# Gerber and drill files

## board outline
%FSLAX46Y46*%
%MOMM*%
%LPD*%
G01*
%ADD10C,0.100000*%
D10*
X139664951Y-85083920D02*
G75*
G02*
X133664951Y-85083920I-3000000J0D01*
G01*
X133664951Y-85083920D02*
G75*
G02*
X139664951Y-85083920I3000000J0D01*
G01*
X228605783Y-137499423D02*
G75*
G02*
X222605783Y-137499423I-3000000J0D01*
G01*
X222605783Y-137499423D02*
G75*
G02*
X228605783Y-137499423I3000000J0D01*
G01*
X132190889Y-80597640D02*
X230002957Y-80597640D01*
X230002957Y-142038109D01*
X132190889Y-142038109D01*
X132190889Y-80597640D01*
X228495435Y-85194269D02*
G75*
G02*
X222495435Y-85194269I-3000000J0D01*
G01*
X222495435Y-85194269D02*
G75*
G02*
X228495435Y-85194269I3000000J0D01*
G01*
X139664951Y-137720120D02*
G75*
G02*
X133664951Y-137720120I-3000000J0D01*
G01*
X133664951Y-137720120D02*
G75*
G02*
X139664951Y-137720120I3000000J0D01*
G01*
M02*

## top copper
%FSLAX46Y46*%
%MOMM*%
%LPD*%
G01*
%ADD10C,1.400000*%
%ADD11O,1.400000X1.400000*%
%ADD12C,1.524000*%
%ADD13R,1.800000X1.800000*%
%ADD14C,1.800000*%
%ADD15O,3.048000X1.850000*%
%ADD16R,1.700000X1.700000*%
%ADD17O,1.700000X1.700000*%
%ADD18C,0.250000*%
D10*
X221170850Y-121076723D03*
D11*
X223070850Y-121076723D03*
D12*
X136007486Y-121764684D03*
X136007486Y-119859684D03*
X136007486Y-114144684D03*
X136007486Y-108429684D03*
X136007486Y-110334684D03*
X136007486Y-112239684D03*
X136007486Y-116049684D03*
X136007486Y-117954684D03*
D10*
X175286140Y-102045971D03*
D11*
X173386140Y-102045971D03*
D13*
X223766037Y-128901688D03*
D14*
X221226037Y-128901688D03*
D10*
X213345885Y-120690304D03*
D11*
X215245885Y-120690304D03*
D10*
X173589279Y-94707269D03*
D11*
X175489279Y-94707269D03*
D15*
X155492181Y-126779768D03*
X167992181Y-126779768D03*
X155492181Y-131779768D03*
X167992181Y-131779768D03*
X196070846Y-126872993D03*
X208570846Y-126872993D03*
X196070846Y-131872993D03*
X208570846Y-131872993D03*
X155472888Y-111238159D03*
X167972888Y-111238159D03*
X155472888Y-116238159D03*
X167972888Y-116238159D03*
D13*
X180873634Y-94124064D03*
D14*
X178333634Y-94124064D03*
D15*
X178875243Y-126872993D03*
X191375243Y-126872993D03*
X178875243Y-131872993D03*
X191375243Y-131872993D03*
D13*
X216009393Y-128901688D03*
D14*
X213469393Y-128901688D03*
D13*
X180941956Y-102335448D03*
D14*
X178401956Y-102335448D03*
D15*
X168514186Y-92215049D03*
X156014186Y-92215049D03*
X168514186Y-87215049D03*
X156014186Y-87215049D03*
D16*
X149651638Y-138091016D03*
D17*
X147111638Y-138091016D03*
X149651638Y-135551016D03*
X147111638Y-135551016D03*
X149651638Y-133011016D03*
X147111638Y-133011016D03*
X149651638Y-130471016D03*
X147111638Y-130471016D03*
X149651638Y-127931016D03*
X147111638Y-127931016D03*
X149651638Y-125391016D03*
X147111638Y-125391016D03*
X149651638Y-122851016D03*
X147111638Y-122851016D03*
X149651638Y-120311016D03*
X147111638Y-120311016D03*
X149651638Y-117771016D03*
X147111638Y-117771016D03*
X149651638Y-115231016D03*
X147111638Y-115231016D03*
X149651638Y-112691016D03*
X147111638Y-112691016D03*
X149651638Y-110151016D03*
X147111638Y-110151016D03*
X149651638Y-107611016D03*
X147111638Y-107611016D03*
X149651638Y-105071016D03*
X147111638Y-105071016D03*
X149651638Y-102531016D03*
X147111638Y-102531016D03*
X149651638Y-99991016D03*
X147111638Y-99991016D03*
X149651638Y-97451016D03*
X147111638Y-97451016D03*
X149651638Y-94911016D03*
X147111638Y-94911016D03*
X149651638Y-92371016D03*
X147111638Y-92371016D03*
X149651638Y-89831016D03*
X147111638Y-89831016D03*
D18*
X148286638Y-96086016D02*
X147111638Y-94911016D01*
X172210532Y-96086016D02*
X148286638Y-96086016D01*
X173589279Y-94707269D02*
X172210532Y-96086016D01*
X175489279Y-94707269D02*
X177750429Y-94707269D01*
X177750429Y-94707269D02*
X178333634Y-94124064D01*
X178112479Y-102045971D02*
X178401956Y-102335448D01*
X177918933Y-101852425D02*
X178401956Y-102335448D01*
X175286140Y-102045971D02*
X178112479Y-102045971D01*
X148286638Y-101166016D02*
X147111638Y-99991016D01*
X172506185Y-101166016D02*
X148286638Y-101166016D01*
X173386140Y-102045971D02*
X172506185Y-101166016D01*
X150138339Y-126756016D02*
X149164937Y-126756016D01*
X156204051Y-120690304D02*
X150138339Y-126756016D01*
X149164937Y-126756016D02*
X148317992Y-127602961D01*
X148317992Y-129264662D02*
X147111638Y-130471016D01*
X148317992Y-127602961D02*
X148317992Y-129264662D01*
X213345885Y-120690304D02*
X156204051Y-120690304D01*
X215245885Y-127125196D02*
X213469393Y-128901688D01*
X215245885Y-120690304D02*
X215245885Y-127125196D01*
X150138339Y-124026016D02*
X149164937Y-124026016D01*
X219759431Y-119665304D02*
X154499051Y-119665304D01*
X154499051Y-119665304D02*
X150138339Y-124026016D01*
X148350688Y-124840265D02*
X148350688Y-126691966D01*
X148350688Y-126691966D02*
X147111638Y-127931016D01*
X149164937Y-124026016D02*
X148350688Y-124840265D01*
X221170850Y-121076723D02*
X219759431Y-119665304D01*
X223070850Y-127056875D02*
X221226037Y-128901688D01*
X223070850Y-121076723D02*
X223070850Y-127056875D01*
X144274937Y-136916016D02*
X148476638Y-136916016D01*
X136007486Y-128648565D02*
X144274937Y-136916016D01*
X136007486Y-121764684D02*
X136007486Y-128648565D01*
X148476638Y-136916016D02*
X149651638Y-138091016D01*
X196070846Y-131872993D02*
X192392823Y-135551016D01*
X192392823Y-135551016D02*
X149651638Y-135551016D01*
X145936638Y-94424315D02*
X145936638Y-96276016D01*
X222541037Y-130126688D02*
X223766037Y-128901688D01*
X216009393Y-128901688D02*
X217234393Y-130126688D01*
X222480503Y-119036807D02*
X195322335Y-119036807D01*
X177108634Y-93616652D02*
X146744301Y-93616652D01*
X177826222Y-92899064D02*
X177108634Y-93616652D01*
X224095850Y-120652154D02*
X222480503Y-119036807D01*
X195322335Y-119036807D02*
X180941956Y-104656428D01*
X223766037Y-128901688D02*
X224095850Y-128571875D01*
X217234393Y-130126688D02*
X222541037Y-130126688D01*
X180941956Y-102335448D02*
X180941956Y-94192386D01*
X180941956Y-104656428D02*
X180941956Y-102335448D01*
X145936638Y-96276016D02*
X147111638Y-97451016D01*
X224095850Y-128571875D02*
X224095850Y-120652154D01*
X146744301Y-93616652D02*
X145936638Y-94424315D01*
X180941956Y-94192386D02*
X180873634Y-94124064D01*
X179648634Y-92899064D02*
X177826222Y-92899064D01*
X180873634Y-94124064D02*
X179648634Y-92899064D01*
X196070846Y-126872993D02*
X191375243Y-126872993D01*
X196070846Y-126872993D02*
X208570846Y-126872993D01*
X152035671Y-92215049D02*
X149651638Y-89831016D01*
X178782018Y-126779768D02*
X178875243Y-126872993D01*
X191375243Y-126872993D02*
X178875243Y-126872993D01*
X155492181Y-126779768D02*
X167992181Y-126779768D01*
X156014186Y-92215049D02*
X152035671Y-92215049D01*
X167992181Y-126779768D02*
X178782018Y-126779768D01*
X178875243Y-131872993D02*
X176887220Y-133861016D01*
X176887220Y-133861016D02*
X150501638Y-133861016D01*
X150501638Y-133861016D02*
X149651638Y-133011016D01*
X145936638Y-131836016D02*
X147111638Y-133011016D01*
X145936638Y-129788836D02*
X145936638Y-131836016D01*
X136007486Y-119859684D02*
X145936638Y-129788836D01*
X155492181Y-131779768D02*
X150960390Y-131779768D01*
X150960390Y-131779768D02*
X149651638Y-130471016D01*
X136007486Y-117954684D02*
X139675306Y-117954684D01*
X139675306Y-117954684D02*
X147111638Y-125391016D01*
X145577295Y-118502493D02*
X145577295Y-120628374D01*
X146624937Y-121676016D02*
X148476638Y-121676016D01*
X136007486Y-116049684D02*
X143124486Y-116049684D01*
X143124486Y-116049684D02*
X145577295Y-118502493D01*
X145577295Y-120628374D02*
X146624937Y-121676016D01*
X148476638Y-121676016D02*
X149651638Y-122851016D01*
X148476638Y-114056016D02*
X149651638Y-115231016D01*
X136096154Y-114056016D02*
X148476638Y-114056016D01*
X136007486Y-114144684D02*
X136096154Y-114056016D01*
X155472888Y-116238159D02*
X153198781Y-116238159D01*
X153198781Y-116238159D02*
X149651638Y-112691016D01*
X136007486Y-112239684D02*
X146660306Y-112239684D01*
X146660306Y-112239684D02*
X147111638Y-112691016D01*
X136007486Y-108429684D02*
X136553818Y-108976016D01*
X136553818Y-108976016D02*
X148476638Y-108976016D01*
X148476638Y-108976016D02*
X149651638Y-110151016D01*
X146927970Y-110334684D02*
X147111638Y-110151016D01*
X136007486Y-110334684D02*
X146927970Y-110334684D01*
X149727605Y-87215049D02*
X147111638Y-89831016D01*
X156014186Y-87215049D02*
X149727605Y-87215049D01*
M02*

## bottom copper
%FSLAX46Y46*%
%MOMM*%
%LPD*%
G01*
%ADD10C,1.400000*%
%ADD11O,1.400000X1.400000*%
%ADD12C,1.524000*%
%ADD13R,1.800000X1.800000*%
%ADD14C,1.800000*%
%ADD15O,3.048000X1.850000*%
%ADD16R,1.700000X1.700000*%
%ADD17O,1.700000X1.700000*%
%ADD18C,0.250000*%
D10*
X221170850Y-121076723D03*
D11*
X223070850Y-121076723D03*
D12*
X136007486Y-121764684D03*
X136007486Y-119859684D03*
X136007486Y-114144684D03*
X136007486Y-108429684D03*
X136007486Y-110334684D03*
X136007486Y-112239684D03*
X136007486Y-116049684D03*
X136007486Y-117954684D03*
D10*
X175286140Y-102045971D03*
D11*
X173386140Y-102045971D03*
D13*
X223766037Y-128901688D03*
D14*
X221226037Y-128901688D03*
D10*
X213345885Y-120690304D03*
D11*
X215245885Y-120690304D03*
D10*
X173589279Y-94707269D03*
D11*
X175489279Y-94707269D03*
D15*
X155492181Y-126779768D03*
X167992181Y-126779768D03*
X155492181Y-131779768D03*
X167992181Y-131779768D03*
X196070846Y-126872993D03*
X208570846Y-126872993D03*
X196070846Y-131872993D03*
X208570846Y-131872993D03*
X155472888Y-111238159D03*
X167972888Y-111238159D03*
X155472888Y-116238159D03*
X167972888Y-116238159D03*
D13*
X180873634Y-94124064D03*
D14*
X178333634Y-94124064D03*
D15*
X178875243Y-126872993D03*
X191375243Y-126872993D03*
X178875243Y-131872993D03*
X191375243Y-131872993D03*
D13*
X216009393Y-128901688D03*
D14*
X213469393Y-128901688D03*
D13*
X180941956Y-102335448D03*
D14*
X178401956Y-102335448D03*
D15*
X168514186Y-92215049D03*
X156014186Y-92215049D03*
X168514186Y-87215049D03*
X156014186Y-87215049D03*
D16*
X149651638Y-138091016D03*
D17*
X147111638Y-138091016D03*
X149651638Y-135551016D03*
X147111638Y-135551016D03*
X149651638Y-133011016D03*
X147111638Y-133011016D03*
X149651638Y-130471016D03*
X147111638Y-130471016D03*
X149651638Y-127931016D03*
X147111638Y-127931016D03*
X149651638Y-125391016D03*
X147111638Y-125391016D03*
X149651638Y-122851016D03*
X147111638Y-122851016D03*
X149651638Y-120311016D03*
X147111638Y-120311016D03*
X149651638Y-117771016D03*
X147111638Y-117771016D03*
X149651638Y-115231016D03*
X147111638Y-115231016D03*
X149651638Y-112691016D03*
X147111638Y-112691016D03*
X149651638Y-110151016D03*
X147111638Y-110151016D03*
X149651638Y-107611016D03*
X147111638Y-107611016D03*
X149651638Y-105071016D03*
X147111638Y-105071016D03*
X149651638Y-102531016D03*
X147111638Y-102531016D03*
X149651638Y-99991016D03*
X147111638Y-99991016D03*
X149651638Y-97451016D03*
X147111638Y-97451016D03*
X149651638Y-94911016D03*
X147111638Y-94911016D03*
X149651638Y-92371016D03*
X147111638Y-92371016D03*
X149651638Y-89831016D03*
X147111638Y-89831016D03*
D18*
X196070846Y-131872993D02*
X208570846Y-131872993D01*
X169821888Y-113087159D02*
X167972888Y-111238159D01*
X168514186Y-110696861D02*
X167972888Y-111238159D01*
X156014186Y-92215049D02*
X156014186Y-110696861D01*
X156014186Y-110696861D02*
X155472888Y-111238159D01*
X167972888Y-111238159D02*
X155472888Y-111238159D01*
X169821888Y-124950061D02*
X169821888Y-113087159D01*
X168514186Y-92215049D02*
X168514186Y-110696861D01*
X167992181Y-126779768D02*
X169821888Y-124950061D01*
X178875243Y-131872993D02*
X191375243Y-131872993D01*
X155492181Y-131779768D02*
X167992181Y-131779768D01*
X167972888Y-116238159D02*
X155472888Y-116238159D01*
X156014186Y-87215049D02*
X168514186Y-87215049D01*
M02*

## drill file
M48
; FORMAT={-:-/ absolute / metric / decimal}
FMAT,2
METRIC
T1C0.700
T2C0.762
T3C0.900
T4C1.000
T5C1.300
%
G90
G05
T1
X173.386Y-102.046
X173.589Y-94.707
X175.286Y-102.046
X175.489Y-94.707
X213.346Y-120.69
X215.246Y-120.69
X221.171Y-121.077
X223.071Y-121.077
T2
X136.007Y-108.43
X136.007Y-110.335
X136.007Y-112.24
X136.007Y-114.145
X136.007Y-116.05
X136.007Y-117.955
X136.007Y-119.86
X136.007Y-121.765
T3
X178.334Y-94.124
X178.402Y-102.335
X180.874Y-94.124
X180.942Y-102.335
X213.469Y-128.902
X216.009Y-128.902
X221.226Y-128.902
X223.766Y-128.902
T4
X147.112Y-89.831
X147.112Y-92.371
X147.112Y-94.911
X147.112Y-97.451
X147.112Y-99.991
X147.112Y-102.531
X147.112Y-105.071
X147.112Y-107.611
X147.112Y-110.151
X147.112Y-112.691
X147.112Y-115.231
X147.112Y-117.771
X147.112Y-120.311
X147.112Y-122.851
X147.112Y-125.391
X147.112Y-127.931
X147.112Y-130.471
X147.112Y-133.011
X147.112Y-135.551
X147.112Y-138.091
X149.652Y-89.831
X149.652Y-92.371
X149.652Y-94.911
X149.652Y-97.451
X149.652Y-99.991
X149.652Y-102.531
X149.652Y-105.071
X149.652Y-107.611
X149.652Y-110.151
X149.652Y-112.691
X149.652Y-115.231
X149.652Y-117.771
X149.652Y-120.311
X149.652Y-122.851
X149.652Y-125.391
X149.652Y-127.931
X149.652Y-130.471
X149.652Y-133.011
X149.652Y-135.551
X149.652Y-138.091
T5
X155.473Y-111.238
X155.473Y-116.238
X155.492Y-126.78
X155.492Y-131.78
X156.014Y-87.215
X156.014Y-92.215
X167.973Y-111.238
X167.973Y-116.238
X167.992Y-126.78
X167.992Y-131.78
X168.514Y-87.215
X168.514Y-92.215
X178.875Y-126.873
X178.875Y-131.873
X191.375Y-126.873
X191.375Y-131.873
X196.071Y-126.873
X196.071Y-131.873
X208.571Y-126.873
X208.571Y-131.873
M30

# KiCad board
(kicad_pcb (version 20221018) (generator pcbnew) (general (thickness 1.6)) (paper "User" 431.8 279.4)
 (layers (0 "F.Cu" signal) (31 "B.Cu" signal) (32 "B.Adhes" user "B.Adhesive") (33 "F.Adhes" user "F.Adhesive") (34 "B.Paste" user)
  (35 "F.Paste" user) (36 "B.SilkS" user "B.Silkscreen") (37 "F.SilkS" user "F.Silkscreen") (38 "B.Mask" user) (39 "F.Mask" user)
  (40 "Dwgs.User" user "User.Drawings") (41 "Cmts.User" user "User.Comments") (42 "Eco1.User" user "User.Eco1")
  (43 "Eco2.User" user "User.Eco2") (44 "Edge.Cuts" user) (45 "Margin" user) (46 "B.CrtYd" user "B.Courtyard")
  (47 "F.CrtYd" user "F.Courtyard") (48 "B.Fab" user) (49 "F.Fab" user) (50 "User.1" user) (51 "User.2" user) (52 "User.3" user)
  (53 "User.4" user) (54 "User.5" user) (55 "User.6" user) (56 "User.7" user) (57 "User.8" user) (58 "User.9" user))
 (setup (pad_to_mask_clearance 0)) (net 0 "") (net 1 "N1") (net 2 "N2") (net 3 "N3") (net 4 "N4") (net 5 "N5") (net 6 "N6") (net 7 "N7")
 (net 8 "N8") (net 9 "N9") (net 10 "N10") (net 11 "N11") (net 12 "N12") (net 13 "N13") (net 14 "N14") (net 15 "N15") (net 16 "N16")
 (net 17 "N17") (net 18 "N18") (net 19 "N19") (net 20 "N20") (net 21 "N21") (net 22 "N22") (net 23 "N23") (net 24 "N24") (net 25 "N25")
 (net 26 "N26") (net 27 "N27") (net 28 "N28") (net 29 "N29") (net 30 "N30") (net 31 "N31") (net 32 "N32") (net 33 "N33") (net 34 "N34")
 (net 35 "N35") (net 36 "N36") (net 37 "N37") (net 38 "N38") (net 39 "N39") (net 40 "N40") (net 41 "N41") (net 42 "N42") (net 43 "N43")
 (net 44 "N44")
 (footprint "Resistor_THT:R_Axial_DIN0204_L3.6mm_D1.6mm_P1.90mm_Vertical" (layer "F.Cu") (at 221.17085 121.076723)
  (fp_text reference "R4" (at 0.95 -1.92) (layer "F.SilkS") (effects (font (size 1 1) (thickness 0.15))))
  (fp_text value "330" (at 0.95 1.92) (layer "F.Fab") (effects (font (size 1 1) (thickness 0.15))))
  (pad "1" thru_hole circle (at 0 0) (size 1.4 1.4) (drill 0.7) (layers "*.Cu" "*.Mask") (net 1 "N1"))
  (pad "2" thru_hole oval (at 1.9 0) (size 1.4 1.4) (drill 0.7) (layers "*.Cu" "*.Mask") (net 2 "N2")))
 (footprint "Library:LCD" (layer "F.Cu") (at 136.007486 117.319684)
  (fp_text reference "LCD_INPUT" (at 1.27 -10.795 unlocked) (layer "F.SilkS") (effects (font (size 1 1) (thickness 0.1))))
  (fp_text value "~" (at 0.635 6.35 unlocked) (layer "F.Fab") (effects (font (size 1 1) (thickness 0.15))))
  (pad "1" thru_hole circle (at 0 4.445) (size 1.524 1.524) (drill 0.762) (layers "*.Cu" "*.Mask") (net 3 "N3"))
  (pad "2" thru_hole circle (at 0 2.54) (size 1.524 1.524) (drill 0.762) (layers "*.Cu" "*.Mask") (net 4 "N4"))
  (pad "3" thru_hole circle (at 0 -3.175) (size 1.524 1.524) (drill 0.762) (layers "*.Cu" "*.Mask") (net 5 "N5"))
  (pad "4" thru_hole circle (at 0 -8.89) (size 1.524 1.524) (drill 0.762) (layers "*.Cu" "*.Mask") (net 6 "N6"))
  (pad "5" thru_hole circle (at 0 -6.985) (size 1.524 1.524) (drill 0.762) (layers "*.Cu" "*.Mask") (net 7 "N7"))
  (pad "6" thru_hole circle (at 0 -5.08) (size 1.524 1.524) (drill 0.762) (layers "*.Cu" "*.Mask") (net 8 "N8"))
  (pad "7" thru_hole circle (at 0 -1.27) (size 1.524 1.524) (drill 0.762) (layers "*.Cu" "*.Mask") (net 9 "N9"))
  (pad "8" thru_hole circle (at 0 0.635) (size 1.524 1.524) (drill 0.762) (layers "*.Cu" "*.Mask") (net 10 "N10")))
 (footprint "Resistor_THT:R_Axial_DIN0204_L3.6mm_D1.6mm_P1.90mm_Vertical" (layer "F.Cu") (at 175.28614 102.045971 180)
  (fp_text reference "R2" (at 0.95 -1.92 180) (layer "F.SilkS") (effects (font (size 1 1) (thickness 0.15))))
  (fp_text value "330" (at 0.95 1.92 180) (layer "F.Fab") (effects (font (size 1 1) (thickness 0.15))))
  (pad "1" thru_hole circle (at 0 0 180) (size 1.4 1.4) (drill 0.7) (layers "*.Cu" "*.Mask") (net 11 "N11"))
  (pad "2" thru_hole oval (at 1.9 0 180) (size 1.4 1.4) (drill 0.7) (layers "*.Cu" "*.Mask") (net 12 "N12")))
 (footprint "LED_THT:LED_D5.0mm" (layer "F.Cu") (at 223.766037 128.901688 180)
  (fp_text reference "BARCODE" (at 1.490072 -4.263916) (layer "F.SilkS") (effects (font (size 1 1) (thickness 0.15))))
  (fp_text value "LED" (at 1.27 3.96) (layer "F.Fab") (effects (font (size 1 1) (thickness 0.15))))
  (pad "1" thru_hole rect (at 0 0 180) (size 1.8 1.8) (drill 0.9) (layers "*.Cu" "*.Mask") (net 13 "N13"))
  (pad "2" thru_hole circle (at 2.54 0 180) (size 1.8 1.8) (drill 0.9) (layers "*.Cu" "*.Mask") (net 2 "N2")))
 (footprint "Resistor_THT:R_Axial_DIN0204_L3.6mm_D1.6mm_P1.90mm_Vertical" (layer "F.Cu") (at 213.345885 120.690304)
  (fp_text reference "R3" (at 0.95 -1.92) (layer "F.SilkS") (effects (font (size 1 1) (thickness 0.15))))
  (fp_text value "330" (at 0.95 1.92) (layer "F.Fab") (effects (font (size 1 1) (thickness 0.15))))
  (pad "1" thru_hole circle (at 0 0) (size 1.4 1.4) (drill 0.7) (layers "*.Cu" "*.Mask") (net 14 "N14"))
  (pad "2" thru_hole oval (at 1.9 0) (size 1.4 1.4) (drill 0.7) (layers "*.Cu" "*.Mask") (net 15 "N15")))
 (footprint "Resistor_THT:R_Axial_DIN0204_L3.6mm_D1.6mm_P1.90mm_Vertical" (layer "F.Cu") (at 173.589279 94.707269)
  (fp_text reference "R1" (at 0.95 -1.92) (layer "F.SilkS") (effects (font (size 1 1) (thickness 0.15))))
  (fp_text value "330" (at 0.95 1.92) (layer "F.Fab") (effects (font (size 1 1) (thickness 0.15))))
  (pad "1" thru_hole circle (at 0 0) (size 1.4 1.4) (drill 0.7) (layers "*.Cu" "*.Mask") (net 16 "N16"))
  (pad "2" thru_hole oval (at 1.9 0) (size 1.4 1.4) (drill 0.7) (layers "*.Cu" "*.Mask") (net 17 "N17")))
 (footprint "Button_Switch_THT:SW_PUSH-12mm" (layer "F.Cu") (at 155.492181 126.779768)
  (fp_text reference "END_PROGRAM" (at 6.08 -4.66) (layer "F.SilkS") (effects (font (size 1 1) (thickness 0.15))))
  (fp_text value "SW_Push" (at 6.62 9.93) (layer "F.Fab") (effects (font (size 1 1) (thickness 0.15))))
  (pad "1" thru_hole oval (at 0 0) (size 3.048 1.85) (drill 1.3) (layers "*.Cu" "*.Mask") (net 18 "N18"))
  (pad "1" thru_hole oval (at 12.5 0) (size 3.048 1.85) (drill 1.3) (layers "*.Cu" "*.Mask") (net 18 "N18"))
  (pad "2" thru_hole oval (at 0 5) (size 3.048 1.85) (drill 1.3) (layers "*.Cu" "*.Mask") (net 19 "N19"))
  (pad "2" thru_hole oval (at 12.5 5) (size 3.048 1.85) (drill 1.3) (layers "*.Cu" "*.Mask") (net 19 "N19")))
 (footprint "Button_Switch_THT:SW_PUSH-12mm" (layer "F.Cu") (at 196.070846 126.872993)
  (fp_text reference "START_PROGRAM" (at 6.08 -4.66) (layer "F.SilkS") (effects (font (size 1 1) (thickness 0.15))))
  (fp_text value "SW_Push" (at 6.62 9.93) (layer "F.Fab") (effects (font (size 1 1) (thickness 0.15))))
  (pad "1" thru_hole oval (at 0 0) (size 3.048 1.85) (drill 1.3) (layers "*.Cu" "*.Mask") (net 18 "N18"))
  (pad "1" thru_hole oval (at 12.5 0) (size 3.048 1.85) (drill 1.3) (layers "*.Cu" "*.Mask") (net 18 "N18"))
  (pad "2" thru_hole oval (at 0 5) (size 3.048 1.85) (drill 1.3) (layers "*.Cu" "*.Mask") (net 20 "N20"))
  (pad "2" thru_hole oval (at 12.5 5) (size 3.048 1.85) (drill 1.3) (layers "*.Cu" "*.Mask") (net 20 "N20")))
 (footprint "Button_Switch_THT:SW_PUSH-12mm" (layer "F.Cu") (at 155.472888 111.238159)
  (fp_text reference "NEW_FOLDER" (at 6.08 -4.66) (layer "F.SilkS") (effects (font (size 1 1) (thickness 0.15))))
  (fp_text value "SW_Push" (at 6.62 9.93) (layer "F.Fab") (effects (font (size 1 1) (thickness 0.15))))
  (pad "1" thru_hole oval (at 0 0) (size 3.048 1.85) (drill 1.3) (layers "*.Cu" "*.Mask") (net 18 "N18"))
  (pad "1" thru_hole oval (at 12.5 0) (size 3.048 1.85) (drill 1.3) (layers "*.Cu" "*.Mask") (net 18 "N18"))
  (pad "2" thru_hole oval (at 0 5) (size 3.048 1.85) (drill 1.3) (layers "*.Cu" "*.Mask") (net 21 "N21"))
  (pad "2" thru_hole oval (at 12.5 5) (size 3.048 1.85) (drill 1.3) (layers "*.Cu" "*.Mask") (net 21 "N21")))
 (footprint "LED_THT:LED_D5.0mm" (layer "F.Cu") (at 180.873634 94.124064 180)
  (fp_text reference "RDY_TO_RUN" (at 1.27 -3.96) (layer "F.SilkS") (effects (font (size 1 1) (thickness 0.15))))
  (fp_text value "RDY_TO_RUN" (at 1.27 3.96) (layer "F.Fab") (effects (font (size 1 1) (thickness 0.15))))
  (pad "1" thru_hole rect (at 0 0 180) (size 1.8 1.8) (drill 0.9) (layers "*.Cu" "*.Mask") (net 13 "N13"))
  (pad "2" thru_hole circle (at 2.54 0 180) (size 1.8 1.8) (drill 0.9) (layers "*.Cu" "*.Mask") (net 17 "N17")))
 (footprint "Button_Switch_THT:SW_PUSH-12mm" (layer "F.Cu") (at 178.875243 126.872993)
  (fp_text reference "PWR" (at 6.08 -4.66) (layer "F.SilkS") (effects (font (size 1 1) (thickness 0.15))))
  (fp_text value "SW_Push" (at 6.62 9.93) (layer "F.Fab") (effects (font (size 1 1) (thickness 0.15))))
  (pad "1" thru_hole oval (at 0 0) (size 3.048 1.85) (drill 1.3) (layers "*.Cu" "*.Mask") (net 18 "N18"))
  (pad "1" thru_hole oval (at 12.5 0) (size 3.048 1.85) (drill 1.3) (layers "*.Cu" "*.Mask") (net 18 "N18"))
  (pad "2" thru_hole oval (at 0 5) (size 3.048 1.85) (drill 1.3) (layers "*.Cu" "*.Mask") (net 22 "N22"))
  (pad "2" thru_hole oval (at 12.5 5) (size 3.048 1.85) (drill 1.3) (layers "*.Cu" "*.Mask") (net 22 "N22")))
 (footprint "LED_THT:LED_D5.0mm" (layer "F.Cu") (at 216.009393 128.901688 180)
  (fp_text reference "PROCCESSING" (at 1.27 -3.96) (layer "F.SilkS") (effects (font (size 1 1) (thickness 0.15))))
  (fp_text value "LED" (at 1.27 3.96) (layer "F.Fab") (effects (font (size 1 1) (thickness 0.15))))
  (pad "1" thru_hole rect (at 0 0 180) (size 1.8 1.8) (drill 0.9) (layers "*.Cu" "*.Mask") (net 13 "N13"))
  (pad "2" thru_hole circle (at 2.54 0 180) (size 1.8 1.8) (drill 0.9) (layers "*.Cu" "*.Mask") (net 15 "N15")))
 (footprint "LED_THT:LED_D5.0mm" (layer "F.Cu") (at 180.941956 102.335448 180)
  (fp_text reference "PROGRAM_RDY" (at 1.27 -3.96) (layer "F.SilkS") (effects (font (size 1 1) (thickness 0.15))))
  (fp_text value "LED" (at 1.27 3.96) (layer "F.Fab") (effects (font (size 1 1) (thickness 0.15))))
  (pad "1" thru_hole rect (at 0 0 180) (size 1.8 1.8) (drill 0.9) (layers "*.Cu" "*.Mask") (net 13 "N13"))
  (pad "2" thru_hole circle (at 2.54 0 180) (size 1.8 1.8) (drill 0.9) (layers "*.Cu" "*.Mask") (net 11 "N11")))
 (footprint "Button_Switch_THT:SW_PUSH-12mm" (layer "F.Cu") (at 168.514186 92.215049 180)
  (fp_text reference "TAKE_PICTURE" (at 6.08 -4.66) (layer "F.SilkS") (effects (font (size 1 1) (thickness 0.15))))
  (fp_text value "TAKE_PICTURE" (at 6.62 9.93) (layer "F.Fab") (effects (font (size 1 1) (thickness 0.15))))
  (pad "1" thru_hole oval (at 0 0 180) (size 3.048 1.85) (drill 1.3) (layers "*.Cu" "*.Mask") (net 18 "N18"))
  (pad "1" thru_hole oval (at 12.5 0 180) (size 3.048 1.85) (drill 1.3) (layers "*.Cu" "*.Mask") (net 18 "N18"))
  (pad "2" thru_hole oval (at 0 5 180) (size 3.048 1.85) (drill 1.3) (layers "*.Cu" "*.Mask") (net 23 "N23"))
  (pad "2" thru_hole oval (at 12.5 5 180) (size 3.048 1.85) (drill 1.3) (layers "*.Cu" "*.Mask") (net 23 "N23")))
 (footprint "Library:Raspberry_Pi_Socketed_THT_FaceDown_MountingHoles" (layer "B.Cu") (at 149.651638 138.091016)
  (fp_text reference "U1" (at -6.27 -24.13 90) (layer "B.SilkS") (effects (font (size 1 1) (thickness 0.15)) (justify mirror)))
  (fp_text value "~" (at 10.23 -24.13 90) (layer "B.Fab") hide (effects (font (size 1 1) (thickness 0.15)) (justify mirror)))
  (pad "1" thru_hole rect (at 0 0) (size 1.7 1.7) (drill 1) (layers "*.Cu" "*.Mask") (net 3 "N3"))
  (pad "2" thru_hole oval (at -2.54 0) (size 1.7 1.7) (drill 1) (layers "*.Cu" "*.Mask") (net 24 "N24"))
  (pad "3" thru_hole oval (at 0 -2.54) (size 1.7 1.7) (drill 1) (layers "*.Cu" "*.Mask") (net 20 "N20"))
  (pad "4" thru_hole oval (at -2.54 -2.54) (size 1.7 1.7) (drill 1) (layers "*.Cu" "*.Mask") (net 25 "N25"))
  (pad "5" thru_hole oval (at 0 -5.08) (size 1.7 1.7) (drill 1) (layers "*.Cu" "*.Mask") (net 22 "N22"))
  (pad "6" thru_hole oval (at -2.54 -5.08) (size 1.7 1.7) (drill 1) (layers "*.Cu" "*.Mask") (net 4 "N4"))
  (pad "7" thru_hole oval (at 0 -7.62) (size 1.7 1.7) (drill 1) (layers "*.Cu" "*.Mask") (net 19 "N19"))
  (pad "8" thru_hole oval (at -2.54 -7.62) (size 1.7 1.7) (drill 1) (layers "*.Cu" "*.Mask") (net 14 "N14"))
  (pad "9" thru_hole oval (at 0 -10.16) (size 1.7 1.7) (drill 1) (layers "*.Cu" "*.Mask") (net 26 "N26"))
  (pad "10" thru_hole oval (at -2.54 -10.16) (size 1.7 1.7) (drill 1) (layers "*.Cu" "*.Mask") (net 1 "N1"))
  (pad "11" thru_hole oval (at 0 -12.7) (size 1.7 1.7) (drill 1) (layers "*.Cu" "*.Mask") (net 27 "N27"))
  (pad "12" thru_hole oval (at -2.54 -12.7) (size 1.7 1.7) (drill 1) (layers "*.Cu" "*.Mask") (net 10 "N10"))
  (pad "13" thru_hole oval (at 0 -15.24) (size 1.7 1.7) (drill 1) (layers "*.Cu" "*.Mask") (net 9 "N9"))
  (pad "14" thru_hole oval (at -2.54 -15.24) (size 1.7 1.7) (drill 1) (layers "*.Cu" "*.Mask") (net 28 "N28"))
  (pad "15" thru_hole oval (at 0 -17.78) (size 1.7 1.7) (drill 1) (layers "*.Cu" "*.Mask") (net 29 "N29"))
  (pad "16" thru_hole oval (at -2.54 -17.78) (size 1.7 1.7) (drill 1) (layers "*.Cu" "*.Mask") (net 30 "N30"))
  (pad "17" thru_hole oval (at 0 -20.32) (size 1.7 1.7) (drill 1) (layers "*.Cu" "*.Mask") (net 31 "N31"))
  (pad "18" thru_hole oval (at -2.54 -20.32) (size 1.7 1.7) (drill 1) (layers "*.Cu" "*.Mask") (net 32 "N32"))
  (pad "19" thru_hole oval (at 0 -22.86) (size 1.7 1.7) (drill 1) (layers "*.Cu" "*.Mask") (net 5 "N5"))
  (pad "20" thru_hole oval (at -2.54 -22.86) (size 1.7 1.7) (drill 1) (layers "*.Cu" "*.Mask") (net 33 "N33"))
  (pad "21" thru_hole oval (at 0 -25.4) (size 1.7 1.7) (drill 1) (layers "*.Cu" "*.Mask") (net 21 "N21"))
  (pad "22" thru_hole oval (at -2.54 -25.4) (size 1.7 1.7) (drill 1) (layers "*.Cu" "*.Mask") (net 8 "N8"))
  (pad "23" thru_hole oval (at 0 -27.94) (size 1.7 1.7) (drill 1) (layers "*.Cu" "*.Mask") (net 6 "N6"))
  (pad "24" thru_hole oval (at -2.54 -27.94) (size 1.7 1.7) (drill 1) (layers "*.Cu" "*.Mask") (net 7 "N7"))
  (pad "25" thru_hole oval (at 0 -30.48) (size 1.7 1.7) (drill 1) (layers "*.Cu" "*.Mask") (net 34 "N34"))
  (pad "26" thru_hole oval (at -2.54 -30.48) (size 1.7 1.7) (drill 1) (layers "*.Cu" "*.Mask") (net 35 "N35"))
  (pad "27" thru_hole oval (at 0 -33.02) (size 1.7 1.7) (drill 1) (layers "*.Cu" "*.Mask") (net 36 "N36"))
  (pad "28" thru_hole oval (at -2.54 -33.02) (size 1.7 1.7) (drill 1) (layers "*.Cu" "*.Mask") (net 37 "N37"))
  (pad "29" thru_hole oval (at 0 -35.56) (size 1.7 1.7) (drill 1) (layers "*.Cu" "*.Mask") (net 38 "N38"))
  (pad "30" thru_hole oval (at -2.54 -35.56) (size 1.7 1.7) (drill 1) (layers "*.Cu" "*.Mask") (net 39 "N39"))
  (pad "31" thru_hole oval (at 0 -38.1) (size 1.7 1.7) (drill 1) (layers "*.Cu" "*.Mask") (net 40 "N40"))
  (pad "32" thru_hole oval (at -2.54 -38.1) (size 1.7 1.7) (drill 1) (layers "*.Cu" "*.Mask") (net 12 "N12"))
  (pad "33" thru_hole oval (at 0 -40.64) (size 1.7 1.7) (drill 1) (layers "*.Cu" "*.Mask") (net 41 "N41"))
  (pad "34" thru_hole oval (at -2.54 -40.64) (size 1.7 1.7) (drill 1) (layers "*.Cu" "*.Mask") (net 13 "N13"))
  (pad "35" thru_hole oval (at 0 -43.18) (size 1.7 1.7) (drill 1) (layers "*.Cu" "*.Mask") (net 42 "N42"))
  (pad "36" thru_hole oval (at -2.54 -43.18) (size 1.7 1.7) (drill 1) (layers "*.Cu" "*.Mask") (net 16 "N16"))
  (pad "37" thru_hole oval (at 0 -45.72) (size 1.7 1.7) (drill 1) (layers "*.Cu" "*.Mask") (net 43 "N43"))
  (pad "38" thru_hole oval (at -2.54 -45.72) (size 1.7 1.7) (drill 1) (layers "*.Cu" "*.Mask") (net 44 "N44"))
  (pad "39" thru_hole oval (at 0 -48.26) (size 1.7 1.7) (drill 1) (layers "*.Cu" "*.Mask") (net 18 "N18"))
  (pad "40" thru_hole oval (at -2.54 -48.26) (size 1.7 1.7) (drill 1) (layers "*.Cu" "*.Mask") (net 23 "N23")))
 (gr_circle (center 136.664951 85.08392) (end 139.664951 85.08392) (stroke (width 0.1) (type default)) (fill none) (layer "Edge.Cuts"))
 (gr_circle (center 225.605783 137.499423) (end 228.605783 137.499423) (stroke (width 0.1) (type default)) (fill none) (layer "Edge.Cuts"))
 (gr_rect (start 132.190889 80.59764) (end 230.002957 142.038109) (stroke (width 0.1) (type default)) (fill none) (layer "Edge.Cuts"))
 (gr_circle (center 225.495435 85.194269) (end 228.495435 85.194269) (stroke (width 0.1) (type default)) (fill none) (layer "Edge.Cuts"))
 (gr_circle (center 136.664951 137.72012) (end 139.664951 137.72012) (stroke (width 0.1) (type default)) (fill none) (layer "Edge.Cuts"))
 (segment (start 148.286638 96.086016) (end 147.111638 94.911016) (width 0.25) (layer "F.Cu") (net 16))
 (segment (start 172.210532 96.086016) (end 148.286638 96.086016) (width 0.25) (layer "F.Cu") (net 16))
 (segment (start 173.589279 94.707269) (end 172.210532 96.086016) (width 0.25) (layer "F.Cu") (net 16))
 (segment (start 175.489279 94.707269) (end 177.750429 94.707269) (width 0.25) (layer "F.Cu") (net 17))
 (segment (start 177.750429 94.707269) (end 178.333634 94.124064) (width 0.25) (layer "F.Cu") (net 17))
 (segment (start 178.112479 102.045971) (end 178.401956 102.335448) (width 0.25) (layer "F.Cu") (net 11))
 (segment (start 177.918933 101.852425) (end 178.401956 102.335448) (width 0.25) (layer "F.Cu") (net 11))
 (segment (start 175.28614 102.045971) (end 178.112479 102.045971) (width 0.25) (layer "F.Cu") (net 11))
 (segment (start 148.286638 101.166016) (end 147.111638 99.991016) (width 0.25) (layer "F.Cu") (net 12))
 (segment (start 172.506185 101.166016) (end 148.286638 101.166016) (width 0.25) (layer "F.Cu") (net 12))
 (segment (start 173.38614 102.045971) (end 172.506185 101.166016) (width 0.25) (layer "F.Cu") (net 12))
 (segment (start 150.138339 126.756016) (end 149.164937 126.756016) (width 0.25) (layer "F.Cu") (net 14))
 (segment (start 156.204051 120.690304) (end 150.138339 126.756016) (width 0.25) (layer "F.Cu") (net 14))
 (segment (start 149.164937 126.756016) (end 148.317992 127.602961) (width 0.25) (layer "F.Cu") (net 14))
 (segment (start 148.317992 129.264662) (end 147.111638 130.471016) (width 0.25) (layer "F.Cu") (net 14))
 (segment (start 148.317992 127.602961) (end 148.317992 129.264662) (width 0.25) (layer "F.Cu") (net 14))
 (segment (start 213.345885 120.690304) (end 156.204051 120.690304) (width 0.25) (layer "F.Cu") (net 14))
 (segment (start 215.245885 127.125196) (end 213.469393 128.901688) (width 0.25) (layer "F.Cu") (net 15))
 (segment (start 215.245885 120.690304) (end 215.245885 127.125196) (width 0.25) (layer "F.Cu") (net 15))
 (segment (start 150.138339 124.026016) (end 149.164937 124.026016) (width 0.25) (layer "F.Cu") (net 1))
 (segment (start 219.759431 119.665304) (end 154.499051 119.665304) (width 0.25) (layer "F.Cu") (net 1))
 (segment (start 154.499051 119.665304) (end 150.138339 124.026016) (width 0.25) (layer "F.Cu") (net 1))
 (segment (start 148.350688 124.840265) (end 148.350688 126.691966) (width 0.25) (layer "F.Cu") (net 1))
 (segment (start 148.350688 126.691966) (end 147.111638 127.931016) (width 0.25) (layer "F.Cu") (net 1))
 (segment (start 149.164937 124.026016) (end 148.350688 124.840265) (width 0.25) (layer "F.Cu") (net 1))
 (segment (start 221.17085 121.076723) (end 219.759431 119.665304) (width 0.25) (layer "F.Cu") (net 1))
 (segment (start 223.07085 127.056875) (end 221.226037 128.901688) (width 0.25) (layer "F.Cu") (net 2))
 (segment (start 223.07085 121.076723) (end 223.07085 127.056875) (width 0.25) (layer "F.Cu") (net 2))
 (segment (start 144.274937 136.916016) (end 148.476638 136.916016) (width 0.25) (layer "F.Cu") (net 3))
 (segment (start 136.007486 128.648565) (end 144.274937 136.916016) (width 0.25) (layer "F.Cu") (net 3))
 (segment (start 136.007486 121.764684) (end 136.007486 128.648565) (width 0.25) (layer "F.Cu") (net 3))
 (segment (start 148.476638 136.916016) (end 149.651638 138.091016) (width 0.25) (layer "F.Cu") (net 3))
 (segment (start 196.070846 131.872993) (end 192.392823 135.551016) (width 0.25) (layer "F.Cu") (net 20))
 (segment (start 192.392823 135.551016) (end 149.651638 135.551016) (width 0.25) (layer "F.Cu") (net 20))
 (segment (start 196.070846 131.872993) (end 208.570846 131.872993) (width 0.25) (layer "B.Cu") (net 20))
 (segment (start 145.936638 94.424315) (end 145.936638 96.276016) (width 0.25) (layer "F.Cu") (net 13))
 (segment (start 222.541037 130.126688) (end 223.766037 128.901688) (width 0.25) (layer "F.Cu") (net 13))
 (segment (start 216.009393 128.901688) (end 217.234393 130.126688) (width 0.25) (layer "F.Cu") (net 13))
 (segment (start 222.480503 119.036807) (end 195.322335 119.036807) (width 0.25) (layer "F.Cu") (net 13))
 (segment (start 177.108634 93.616652) (end 146.744301 93.616652) (width 0.25) (layer "F.Cu") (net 13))
 (segment (start 177.826222 92.899064) (end 177.108634 93.616652) (width 0.25) (layer "F.Cu") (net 13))
 (segment (start 224.09585 120.652154) (end 222.480503 119.036807) (width 0.25) (layer "F.Cu") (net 13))
 (segment (start 195.322335 119.036807) (end 180.941956 104.656428) (width 0.25) (layer "F.Cu") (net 13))
 (segment (start 223.766037 128.901688) (end 224.09585 128.571875) (width 0.25) (layer "F.Cu") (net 13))
 (segment (start 217.234393 130.126688) (end 222.541037 130.126688) (width 0.25) (layer "F.Cu") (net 13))
 (segment (start 180.941956 102.335448) (end 180.941956 94.192386) (width 0.25) (layer "F.Cu") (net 13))
 (segment (start 180.941956 104.656428) (end 180.941956 102.335448) (width 0.25) (layer "F.Cu") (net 13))
 (segment (start 145.936638 96.276016) (end 147.111638 97.451016) (width 0.25) (layer "F.Cu") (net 13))
 (segment (start 224.09585 128.571875) (end 224.09585 120.652154) (width 0.25) (layer "F.Cu") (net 13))
 (segment (start 146.744301 93.616652) (end 145.936638 94.424315) (width 0.25) (layer "F.Cu") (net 13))
 (segment (start 180.941956 94.192386) (end 180.873634 94.124064) (width 0.25) (layer "F.Cu") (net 13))
 (segment (start 179.648634 92.899064) (end 177.826222 92.899064) (width 0.25) (layer "F.Cu") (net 13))
 (segment (start 180.873634 94.124064) (end 179.648634 92.899064) (width 0.25) (layer "F.Cu") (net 13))
 (segment (start 196.070846 126.872993) (end 191.375243 126.872993) (width 0.25) (layer "F.Cu") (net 18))
 (segment (start 196.070846 126.872993) (end 208.570846 126.872993) (width 0.25) (layer "F.Cu") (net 18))
 (segment (start 152.035671 92.215049) (end 149.651638 89.831016) (width 0.25) (layer "F.Cu") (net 18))
 (segment (start 178.782018 126.779768) (end 178.875243 126.872993) (width 0.25) (layer "F.Cu") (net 18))
 (segment (start 191.375243 126.872993) (end 178.875243 126.872993) (width 0.25) (layer "F.Cu") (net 18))
 (segment (start 155.492181 126.779768) (end 167.992181 126.779768) (width 0.25) (layer "F.Cu") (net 18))
 (segment (start 156.014186 92.215049) (end 152.035671 92.215049) (width 0.25) (layer "F.Cu") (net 18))
 (segment (start 167.992181 126.779768) (end 178.782018 126.779768) (width 0.25) (layer "F.Cu") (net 18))
 (segment (start 169.821888 113.087159) (end 167.972888 111.238159) (width 0.25) (layer "B.Cu") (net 18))
 (segment (start 168.514186 110.696861) (end 167.972888 111.238159) (width 0.25) (layer "B.Cu") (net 18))
 (segment (start 156.014186 92.215049) (end 156.014186 110.696861) (width 0.25) (layer "B.Cu") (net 18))
 (segment (start 156.014186 110.696861) (end 155.472888 111.238159) (width 0.25) (layer "B.Cu") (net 18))
 (segment (start 167.972888 111.238159) (end 155.472888 111.238159) (width 0.25) (layer "B.Cu") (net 18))
 (segment (start 169.821888 124.950061) (end 169.821888 113.087159) (width 0.25) (layer "B.Cu") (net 18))
 (segment (start 168.514186 92.215049) (end 168.514186 110.696861) (width 0.25) (layer "B.Cu") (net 18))
 (segment (start 167.992181 126.779768) (end 169.821888 124.950061) (width 0.25) (layer "B.Cu") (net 18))
 (segment (start 178.875243 131.872993) (end 176.88722 133.861016) (width 0.25) (layer "F.Cu") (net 22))
 (segment (start 176.88722 133.861016) (end 150.501638 133.861016) (width 0.25) (layer "F.Cu") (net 22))
 (segment (start 150.501638 133.861016) (end 149.651638 133.011016) (width 0.25) (layer "F.Cu") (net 22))
 (segment (start 178.875243 131.872993) (end 191.375243 131.872993) (width 0.25) (layer "B.Cu") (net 22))
 (segment (start 145.936638 131.836016) (end 147.111638 133.011016) (width 0.25) (layer "F.Cu") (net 4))
 (segment (start 145.936638 129.788836) (end 145.936638 131.836016) (width 0.25) (layer "F.Cu") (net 4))
 (segment (start 136.007486 119.859684) (end 145.936638 129.788836) (width 0.25) (layer "F.Cu") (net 4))
 (segment (start 155.492181 131.779768) (end 150.96039 131.779768) (width 0.25) (layer "F.Cu") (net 19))
 (segment (start 150.96039 131.779768) (end 149.651638 130.471016) (width 0.25) (layer "F.Cu") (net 19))
 (segment (start 155.492181 131.779768) (end 167.992181 131.779768) (width 0.25) (layer "B.Cu") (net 19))
 (segment (start 136.007486 117.954684) (end 139.675306 117.954684) (width 0.25) (layer "F.Cu") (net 10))
 (segment (start 139.675306 117.954684) (end 147.111638 125.391016) (width 0.25) (layer "F.Cu") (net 10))
 (segment (start 145.577295 118.502493) (end 145.577295 120.628374) (width 0.25) (layer "F.Cu") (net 9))
 (segment (start 146.624937 121.676016) (end 148.476638 121.676016) (width 0.25) (layer "F.Cu") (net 9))
 (segment (start 136.007486 116.049684) (end 143.124486 116.049684) (width 0.25) (layer "F.Cu") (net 9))
 (segment (start 143.124486 116.049684) (end 145.577295 118.502493) (width 0.25) (layer "F.Cu") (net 9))
 (segment (start 145.577295 120.628374) (end 146.624937 121.676016) (width 0.25) (layer "F.Cu") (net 9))
 (segment (start 148.476638 121.676016) (end 149.651638 122.851016) (width 0.25) (layer "F.Cu") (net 9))
 (segment (start 148.476638 114.056016) (end 149.651638 115.231016) (width 0.25) (layer "F.Cu") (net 5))
 (segment (start 136.096154 114.056016) (end 148.476638 114.056016) (width 0.25) (layer "F.Cu") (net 5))
 (segment (start 136.007486 114.144684) (end 136.096154 114.056016) (width 0.25) (layer "F.Cu") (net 5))
 (segment (start 155.472888 116.238159) (end 153.198781 116.238159) (width 0.25) (layer "F.Cu") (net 21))
 (segment (start 153.198781 116.238159) (end 149.651638 112.691016) (width 0.25) (layer "F.Cu") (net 21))
 (segment (start 167.972888 116.238159) (end 155.472888 116.238159) (width 0.25) (layer "B.Cu") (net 21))
 (segment (start 136.007486 112.239684) (end 146.660306 112.239684) (width 0.25) (layer "F.Cu") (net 8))
 (segment (start 146.660306 112.239684) (end 147.111638 112.691016) (width 0.25) (layer "F.Cu") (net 8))
 (segment (start 136.007486 108.429684) (end 136.553818 108.976016) (width 0.25) (layer "F.Cu") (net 6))
 (segment (start 136.553818 108.976016) (end 148.476638 108.976016) (width 0.25) (layer "F.Cu") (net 6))
 (segment (start 148.476638 108.976016) (end 149.651638 110.151016) (width 0.25) (layer "F.Cu") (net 6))
 (segment (start 146.92797 110.334684) (end 147.111638 110.151016) (width 0.25) (layer "F.Cu") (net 7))
 (segment (start 136.007486 110.334684) (end 146.92797 110.334684) (width 0.25) (layer "F.Cu") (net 7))
 (segment (start 149.727605 87.215049) (end 147.111638 89.831016) (width 0.25) (layer "F.Cu") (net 23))
 (segment (start 156.014186 87.215049) (end 149.727605 87.215049) (width 0.25) (layer "F.Cu") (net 23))
 (segment (start 156.014186 87.215049) (end 168.514186 87.215049) (width 0.25) (layer "B.Cu") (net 23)))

